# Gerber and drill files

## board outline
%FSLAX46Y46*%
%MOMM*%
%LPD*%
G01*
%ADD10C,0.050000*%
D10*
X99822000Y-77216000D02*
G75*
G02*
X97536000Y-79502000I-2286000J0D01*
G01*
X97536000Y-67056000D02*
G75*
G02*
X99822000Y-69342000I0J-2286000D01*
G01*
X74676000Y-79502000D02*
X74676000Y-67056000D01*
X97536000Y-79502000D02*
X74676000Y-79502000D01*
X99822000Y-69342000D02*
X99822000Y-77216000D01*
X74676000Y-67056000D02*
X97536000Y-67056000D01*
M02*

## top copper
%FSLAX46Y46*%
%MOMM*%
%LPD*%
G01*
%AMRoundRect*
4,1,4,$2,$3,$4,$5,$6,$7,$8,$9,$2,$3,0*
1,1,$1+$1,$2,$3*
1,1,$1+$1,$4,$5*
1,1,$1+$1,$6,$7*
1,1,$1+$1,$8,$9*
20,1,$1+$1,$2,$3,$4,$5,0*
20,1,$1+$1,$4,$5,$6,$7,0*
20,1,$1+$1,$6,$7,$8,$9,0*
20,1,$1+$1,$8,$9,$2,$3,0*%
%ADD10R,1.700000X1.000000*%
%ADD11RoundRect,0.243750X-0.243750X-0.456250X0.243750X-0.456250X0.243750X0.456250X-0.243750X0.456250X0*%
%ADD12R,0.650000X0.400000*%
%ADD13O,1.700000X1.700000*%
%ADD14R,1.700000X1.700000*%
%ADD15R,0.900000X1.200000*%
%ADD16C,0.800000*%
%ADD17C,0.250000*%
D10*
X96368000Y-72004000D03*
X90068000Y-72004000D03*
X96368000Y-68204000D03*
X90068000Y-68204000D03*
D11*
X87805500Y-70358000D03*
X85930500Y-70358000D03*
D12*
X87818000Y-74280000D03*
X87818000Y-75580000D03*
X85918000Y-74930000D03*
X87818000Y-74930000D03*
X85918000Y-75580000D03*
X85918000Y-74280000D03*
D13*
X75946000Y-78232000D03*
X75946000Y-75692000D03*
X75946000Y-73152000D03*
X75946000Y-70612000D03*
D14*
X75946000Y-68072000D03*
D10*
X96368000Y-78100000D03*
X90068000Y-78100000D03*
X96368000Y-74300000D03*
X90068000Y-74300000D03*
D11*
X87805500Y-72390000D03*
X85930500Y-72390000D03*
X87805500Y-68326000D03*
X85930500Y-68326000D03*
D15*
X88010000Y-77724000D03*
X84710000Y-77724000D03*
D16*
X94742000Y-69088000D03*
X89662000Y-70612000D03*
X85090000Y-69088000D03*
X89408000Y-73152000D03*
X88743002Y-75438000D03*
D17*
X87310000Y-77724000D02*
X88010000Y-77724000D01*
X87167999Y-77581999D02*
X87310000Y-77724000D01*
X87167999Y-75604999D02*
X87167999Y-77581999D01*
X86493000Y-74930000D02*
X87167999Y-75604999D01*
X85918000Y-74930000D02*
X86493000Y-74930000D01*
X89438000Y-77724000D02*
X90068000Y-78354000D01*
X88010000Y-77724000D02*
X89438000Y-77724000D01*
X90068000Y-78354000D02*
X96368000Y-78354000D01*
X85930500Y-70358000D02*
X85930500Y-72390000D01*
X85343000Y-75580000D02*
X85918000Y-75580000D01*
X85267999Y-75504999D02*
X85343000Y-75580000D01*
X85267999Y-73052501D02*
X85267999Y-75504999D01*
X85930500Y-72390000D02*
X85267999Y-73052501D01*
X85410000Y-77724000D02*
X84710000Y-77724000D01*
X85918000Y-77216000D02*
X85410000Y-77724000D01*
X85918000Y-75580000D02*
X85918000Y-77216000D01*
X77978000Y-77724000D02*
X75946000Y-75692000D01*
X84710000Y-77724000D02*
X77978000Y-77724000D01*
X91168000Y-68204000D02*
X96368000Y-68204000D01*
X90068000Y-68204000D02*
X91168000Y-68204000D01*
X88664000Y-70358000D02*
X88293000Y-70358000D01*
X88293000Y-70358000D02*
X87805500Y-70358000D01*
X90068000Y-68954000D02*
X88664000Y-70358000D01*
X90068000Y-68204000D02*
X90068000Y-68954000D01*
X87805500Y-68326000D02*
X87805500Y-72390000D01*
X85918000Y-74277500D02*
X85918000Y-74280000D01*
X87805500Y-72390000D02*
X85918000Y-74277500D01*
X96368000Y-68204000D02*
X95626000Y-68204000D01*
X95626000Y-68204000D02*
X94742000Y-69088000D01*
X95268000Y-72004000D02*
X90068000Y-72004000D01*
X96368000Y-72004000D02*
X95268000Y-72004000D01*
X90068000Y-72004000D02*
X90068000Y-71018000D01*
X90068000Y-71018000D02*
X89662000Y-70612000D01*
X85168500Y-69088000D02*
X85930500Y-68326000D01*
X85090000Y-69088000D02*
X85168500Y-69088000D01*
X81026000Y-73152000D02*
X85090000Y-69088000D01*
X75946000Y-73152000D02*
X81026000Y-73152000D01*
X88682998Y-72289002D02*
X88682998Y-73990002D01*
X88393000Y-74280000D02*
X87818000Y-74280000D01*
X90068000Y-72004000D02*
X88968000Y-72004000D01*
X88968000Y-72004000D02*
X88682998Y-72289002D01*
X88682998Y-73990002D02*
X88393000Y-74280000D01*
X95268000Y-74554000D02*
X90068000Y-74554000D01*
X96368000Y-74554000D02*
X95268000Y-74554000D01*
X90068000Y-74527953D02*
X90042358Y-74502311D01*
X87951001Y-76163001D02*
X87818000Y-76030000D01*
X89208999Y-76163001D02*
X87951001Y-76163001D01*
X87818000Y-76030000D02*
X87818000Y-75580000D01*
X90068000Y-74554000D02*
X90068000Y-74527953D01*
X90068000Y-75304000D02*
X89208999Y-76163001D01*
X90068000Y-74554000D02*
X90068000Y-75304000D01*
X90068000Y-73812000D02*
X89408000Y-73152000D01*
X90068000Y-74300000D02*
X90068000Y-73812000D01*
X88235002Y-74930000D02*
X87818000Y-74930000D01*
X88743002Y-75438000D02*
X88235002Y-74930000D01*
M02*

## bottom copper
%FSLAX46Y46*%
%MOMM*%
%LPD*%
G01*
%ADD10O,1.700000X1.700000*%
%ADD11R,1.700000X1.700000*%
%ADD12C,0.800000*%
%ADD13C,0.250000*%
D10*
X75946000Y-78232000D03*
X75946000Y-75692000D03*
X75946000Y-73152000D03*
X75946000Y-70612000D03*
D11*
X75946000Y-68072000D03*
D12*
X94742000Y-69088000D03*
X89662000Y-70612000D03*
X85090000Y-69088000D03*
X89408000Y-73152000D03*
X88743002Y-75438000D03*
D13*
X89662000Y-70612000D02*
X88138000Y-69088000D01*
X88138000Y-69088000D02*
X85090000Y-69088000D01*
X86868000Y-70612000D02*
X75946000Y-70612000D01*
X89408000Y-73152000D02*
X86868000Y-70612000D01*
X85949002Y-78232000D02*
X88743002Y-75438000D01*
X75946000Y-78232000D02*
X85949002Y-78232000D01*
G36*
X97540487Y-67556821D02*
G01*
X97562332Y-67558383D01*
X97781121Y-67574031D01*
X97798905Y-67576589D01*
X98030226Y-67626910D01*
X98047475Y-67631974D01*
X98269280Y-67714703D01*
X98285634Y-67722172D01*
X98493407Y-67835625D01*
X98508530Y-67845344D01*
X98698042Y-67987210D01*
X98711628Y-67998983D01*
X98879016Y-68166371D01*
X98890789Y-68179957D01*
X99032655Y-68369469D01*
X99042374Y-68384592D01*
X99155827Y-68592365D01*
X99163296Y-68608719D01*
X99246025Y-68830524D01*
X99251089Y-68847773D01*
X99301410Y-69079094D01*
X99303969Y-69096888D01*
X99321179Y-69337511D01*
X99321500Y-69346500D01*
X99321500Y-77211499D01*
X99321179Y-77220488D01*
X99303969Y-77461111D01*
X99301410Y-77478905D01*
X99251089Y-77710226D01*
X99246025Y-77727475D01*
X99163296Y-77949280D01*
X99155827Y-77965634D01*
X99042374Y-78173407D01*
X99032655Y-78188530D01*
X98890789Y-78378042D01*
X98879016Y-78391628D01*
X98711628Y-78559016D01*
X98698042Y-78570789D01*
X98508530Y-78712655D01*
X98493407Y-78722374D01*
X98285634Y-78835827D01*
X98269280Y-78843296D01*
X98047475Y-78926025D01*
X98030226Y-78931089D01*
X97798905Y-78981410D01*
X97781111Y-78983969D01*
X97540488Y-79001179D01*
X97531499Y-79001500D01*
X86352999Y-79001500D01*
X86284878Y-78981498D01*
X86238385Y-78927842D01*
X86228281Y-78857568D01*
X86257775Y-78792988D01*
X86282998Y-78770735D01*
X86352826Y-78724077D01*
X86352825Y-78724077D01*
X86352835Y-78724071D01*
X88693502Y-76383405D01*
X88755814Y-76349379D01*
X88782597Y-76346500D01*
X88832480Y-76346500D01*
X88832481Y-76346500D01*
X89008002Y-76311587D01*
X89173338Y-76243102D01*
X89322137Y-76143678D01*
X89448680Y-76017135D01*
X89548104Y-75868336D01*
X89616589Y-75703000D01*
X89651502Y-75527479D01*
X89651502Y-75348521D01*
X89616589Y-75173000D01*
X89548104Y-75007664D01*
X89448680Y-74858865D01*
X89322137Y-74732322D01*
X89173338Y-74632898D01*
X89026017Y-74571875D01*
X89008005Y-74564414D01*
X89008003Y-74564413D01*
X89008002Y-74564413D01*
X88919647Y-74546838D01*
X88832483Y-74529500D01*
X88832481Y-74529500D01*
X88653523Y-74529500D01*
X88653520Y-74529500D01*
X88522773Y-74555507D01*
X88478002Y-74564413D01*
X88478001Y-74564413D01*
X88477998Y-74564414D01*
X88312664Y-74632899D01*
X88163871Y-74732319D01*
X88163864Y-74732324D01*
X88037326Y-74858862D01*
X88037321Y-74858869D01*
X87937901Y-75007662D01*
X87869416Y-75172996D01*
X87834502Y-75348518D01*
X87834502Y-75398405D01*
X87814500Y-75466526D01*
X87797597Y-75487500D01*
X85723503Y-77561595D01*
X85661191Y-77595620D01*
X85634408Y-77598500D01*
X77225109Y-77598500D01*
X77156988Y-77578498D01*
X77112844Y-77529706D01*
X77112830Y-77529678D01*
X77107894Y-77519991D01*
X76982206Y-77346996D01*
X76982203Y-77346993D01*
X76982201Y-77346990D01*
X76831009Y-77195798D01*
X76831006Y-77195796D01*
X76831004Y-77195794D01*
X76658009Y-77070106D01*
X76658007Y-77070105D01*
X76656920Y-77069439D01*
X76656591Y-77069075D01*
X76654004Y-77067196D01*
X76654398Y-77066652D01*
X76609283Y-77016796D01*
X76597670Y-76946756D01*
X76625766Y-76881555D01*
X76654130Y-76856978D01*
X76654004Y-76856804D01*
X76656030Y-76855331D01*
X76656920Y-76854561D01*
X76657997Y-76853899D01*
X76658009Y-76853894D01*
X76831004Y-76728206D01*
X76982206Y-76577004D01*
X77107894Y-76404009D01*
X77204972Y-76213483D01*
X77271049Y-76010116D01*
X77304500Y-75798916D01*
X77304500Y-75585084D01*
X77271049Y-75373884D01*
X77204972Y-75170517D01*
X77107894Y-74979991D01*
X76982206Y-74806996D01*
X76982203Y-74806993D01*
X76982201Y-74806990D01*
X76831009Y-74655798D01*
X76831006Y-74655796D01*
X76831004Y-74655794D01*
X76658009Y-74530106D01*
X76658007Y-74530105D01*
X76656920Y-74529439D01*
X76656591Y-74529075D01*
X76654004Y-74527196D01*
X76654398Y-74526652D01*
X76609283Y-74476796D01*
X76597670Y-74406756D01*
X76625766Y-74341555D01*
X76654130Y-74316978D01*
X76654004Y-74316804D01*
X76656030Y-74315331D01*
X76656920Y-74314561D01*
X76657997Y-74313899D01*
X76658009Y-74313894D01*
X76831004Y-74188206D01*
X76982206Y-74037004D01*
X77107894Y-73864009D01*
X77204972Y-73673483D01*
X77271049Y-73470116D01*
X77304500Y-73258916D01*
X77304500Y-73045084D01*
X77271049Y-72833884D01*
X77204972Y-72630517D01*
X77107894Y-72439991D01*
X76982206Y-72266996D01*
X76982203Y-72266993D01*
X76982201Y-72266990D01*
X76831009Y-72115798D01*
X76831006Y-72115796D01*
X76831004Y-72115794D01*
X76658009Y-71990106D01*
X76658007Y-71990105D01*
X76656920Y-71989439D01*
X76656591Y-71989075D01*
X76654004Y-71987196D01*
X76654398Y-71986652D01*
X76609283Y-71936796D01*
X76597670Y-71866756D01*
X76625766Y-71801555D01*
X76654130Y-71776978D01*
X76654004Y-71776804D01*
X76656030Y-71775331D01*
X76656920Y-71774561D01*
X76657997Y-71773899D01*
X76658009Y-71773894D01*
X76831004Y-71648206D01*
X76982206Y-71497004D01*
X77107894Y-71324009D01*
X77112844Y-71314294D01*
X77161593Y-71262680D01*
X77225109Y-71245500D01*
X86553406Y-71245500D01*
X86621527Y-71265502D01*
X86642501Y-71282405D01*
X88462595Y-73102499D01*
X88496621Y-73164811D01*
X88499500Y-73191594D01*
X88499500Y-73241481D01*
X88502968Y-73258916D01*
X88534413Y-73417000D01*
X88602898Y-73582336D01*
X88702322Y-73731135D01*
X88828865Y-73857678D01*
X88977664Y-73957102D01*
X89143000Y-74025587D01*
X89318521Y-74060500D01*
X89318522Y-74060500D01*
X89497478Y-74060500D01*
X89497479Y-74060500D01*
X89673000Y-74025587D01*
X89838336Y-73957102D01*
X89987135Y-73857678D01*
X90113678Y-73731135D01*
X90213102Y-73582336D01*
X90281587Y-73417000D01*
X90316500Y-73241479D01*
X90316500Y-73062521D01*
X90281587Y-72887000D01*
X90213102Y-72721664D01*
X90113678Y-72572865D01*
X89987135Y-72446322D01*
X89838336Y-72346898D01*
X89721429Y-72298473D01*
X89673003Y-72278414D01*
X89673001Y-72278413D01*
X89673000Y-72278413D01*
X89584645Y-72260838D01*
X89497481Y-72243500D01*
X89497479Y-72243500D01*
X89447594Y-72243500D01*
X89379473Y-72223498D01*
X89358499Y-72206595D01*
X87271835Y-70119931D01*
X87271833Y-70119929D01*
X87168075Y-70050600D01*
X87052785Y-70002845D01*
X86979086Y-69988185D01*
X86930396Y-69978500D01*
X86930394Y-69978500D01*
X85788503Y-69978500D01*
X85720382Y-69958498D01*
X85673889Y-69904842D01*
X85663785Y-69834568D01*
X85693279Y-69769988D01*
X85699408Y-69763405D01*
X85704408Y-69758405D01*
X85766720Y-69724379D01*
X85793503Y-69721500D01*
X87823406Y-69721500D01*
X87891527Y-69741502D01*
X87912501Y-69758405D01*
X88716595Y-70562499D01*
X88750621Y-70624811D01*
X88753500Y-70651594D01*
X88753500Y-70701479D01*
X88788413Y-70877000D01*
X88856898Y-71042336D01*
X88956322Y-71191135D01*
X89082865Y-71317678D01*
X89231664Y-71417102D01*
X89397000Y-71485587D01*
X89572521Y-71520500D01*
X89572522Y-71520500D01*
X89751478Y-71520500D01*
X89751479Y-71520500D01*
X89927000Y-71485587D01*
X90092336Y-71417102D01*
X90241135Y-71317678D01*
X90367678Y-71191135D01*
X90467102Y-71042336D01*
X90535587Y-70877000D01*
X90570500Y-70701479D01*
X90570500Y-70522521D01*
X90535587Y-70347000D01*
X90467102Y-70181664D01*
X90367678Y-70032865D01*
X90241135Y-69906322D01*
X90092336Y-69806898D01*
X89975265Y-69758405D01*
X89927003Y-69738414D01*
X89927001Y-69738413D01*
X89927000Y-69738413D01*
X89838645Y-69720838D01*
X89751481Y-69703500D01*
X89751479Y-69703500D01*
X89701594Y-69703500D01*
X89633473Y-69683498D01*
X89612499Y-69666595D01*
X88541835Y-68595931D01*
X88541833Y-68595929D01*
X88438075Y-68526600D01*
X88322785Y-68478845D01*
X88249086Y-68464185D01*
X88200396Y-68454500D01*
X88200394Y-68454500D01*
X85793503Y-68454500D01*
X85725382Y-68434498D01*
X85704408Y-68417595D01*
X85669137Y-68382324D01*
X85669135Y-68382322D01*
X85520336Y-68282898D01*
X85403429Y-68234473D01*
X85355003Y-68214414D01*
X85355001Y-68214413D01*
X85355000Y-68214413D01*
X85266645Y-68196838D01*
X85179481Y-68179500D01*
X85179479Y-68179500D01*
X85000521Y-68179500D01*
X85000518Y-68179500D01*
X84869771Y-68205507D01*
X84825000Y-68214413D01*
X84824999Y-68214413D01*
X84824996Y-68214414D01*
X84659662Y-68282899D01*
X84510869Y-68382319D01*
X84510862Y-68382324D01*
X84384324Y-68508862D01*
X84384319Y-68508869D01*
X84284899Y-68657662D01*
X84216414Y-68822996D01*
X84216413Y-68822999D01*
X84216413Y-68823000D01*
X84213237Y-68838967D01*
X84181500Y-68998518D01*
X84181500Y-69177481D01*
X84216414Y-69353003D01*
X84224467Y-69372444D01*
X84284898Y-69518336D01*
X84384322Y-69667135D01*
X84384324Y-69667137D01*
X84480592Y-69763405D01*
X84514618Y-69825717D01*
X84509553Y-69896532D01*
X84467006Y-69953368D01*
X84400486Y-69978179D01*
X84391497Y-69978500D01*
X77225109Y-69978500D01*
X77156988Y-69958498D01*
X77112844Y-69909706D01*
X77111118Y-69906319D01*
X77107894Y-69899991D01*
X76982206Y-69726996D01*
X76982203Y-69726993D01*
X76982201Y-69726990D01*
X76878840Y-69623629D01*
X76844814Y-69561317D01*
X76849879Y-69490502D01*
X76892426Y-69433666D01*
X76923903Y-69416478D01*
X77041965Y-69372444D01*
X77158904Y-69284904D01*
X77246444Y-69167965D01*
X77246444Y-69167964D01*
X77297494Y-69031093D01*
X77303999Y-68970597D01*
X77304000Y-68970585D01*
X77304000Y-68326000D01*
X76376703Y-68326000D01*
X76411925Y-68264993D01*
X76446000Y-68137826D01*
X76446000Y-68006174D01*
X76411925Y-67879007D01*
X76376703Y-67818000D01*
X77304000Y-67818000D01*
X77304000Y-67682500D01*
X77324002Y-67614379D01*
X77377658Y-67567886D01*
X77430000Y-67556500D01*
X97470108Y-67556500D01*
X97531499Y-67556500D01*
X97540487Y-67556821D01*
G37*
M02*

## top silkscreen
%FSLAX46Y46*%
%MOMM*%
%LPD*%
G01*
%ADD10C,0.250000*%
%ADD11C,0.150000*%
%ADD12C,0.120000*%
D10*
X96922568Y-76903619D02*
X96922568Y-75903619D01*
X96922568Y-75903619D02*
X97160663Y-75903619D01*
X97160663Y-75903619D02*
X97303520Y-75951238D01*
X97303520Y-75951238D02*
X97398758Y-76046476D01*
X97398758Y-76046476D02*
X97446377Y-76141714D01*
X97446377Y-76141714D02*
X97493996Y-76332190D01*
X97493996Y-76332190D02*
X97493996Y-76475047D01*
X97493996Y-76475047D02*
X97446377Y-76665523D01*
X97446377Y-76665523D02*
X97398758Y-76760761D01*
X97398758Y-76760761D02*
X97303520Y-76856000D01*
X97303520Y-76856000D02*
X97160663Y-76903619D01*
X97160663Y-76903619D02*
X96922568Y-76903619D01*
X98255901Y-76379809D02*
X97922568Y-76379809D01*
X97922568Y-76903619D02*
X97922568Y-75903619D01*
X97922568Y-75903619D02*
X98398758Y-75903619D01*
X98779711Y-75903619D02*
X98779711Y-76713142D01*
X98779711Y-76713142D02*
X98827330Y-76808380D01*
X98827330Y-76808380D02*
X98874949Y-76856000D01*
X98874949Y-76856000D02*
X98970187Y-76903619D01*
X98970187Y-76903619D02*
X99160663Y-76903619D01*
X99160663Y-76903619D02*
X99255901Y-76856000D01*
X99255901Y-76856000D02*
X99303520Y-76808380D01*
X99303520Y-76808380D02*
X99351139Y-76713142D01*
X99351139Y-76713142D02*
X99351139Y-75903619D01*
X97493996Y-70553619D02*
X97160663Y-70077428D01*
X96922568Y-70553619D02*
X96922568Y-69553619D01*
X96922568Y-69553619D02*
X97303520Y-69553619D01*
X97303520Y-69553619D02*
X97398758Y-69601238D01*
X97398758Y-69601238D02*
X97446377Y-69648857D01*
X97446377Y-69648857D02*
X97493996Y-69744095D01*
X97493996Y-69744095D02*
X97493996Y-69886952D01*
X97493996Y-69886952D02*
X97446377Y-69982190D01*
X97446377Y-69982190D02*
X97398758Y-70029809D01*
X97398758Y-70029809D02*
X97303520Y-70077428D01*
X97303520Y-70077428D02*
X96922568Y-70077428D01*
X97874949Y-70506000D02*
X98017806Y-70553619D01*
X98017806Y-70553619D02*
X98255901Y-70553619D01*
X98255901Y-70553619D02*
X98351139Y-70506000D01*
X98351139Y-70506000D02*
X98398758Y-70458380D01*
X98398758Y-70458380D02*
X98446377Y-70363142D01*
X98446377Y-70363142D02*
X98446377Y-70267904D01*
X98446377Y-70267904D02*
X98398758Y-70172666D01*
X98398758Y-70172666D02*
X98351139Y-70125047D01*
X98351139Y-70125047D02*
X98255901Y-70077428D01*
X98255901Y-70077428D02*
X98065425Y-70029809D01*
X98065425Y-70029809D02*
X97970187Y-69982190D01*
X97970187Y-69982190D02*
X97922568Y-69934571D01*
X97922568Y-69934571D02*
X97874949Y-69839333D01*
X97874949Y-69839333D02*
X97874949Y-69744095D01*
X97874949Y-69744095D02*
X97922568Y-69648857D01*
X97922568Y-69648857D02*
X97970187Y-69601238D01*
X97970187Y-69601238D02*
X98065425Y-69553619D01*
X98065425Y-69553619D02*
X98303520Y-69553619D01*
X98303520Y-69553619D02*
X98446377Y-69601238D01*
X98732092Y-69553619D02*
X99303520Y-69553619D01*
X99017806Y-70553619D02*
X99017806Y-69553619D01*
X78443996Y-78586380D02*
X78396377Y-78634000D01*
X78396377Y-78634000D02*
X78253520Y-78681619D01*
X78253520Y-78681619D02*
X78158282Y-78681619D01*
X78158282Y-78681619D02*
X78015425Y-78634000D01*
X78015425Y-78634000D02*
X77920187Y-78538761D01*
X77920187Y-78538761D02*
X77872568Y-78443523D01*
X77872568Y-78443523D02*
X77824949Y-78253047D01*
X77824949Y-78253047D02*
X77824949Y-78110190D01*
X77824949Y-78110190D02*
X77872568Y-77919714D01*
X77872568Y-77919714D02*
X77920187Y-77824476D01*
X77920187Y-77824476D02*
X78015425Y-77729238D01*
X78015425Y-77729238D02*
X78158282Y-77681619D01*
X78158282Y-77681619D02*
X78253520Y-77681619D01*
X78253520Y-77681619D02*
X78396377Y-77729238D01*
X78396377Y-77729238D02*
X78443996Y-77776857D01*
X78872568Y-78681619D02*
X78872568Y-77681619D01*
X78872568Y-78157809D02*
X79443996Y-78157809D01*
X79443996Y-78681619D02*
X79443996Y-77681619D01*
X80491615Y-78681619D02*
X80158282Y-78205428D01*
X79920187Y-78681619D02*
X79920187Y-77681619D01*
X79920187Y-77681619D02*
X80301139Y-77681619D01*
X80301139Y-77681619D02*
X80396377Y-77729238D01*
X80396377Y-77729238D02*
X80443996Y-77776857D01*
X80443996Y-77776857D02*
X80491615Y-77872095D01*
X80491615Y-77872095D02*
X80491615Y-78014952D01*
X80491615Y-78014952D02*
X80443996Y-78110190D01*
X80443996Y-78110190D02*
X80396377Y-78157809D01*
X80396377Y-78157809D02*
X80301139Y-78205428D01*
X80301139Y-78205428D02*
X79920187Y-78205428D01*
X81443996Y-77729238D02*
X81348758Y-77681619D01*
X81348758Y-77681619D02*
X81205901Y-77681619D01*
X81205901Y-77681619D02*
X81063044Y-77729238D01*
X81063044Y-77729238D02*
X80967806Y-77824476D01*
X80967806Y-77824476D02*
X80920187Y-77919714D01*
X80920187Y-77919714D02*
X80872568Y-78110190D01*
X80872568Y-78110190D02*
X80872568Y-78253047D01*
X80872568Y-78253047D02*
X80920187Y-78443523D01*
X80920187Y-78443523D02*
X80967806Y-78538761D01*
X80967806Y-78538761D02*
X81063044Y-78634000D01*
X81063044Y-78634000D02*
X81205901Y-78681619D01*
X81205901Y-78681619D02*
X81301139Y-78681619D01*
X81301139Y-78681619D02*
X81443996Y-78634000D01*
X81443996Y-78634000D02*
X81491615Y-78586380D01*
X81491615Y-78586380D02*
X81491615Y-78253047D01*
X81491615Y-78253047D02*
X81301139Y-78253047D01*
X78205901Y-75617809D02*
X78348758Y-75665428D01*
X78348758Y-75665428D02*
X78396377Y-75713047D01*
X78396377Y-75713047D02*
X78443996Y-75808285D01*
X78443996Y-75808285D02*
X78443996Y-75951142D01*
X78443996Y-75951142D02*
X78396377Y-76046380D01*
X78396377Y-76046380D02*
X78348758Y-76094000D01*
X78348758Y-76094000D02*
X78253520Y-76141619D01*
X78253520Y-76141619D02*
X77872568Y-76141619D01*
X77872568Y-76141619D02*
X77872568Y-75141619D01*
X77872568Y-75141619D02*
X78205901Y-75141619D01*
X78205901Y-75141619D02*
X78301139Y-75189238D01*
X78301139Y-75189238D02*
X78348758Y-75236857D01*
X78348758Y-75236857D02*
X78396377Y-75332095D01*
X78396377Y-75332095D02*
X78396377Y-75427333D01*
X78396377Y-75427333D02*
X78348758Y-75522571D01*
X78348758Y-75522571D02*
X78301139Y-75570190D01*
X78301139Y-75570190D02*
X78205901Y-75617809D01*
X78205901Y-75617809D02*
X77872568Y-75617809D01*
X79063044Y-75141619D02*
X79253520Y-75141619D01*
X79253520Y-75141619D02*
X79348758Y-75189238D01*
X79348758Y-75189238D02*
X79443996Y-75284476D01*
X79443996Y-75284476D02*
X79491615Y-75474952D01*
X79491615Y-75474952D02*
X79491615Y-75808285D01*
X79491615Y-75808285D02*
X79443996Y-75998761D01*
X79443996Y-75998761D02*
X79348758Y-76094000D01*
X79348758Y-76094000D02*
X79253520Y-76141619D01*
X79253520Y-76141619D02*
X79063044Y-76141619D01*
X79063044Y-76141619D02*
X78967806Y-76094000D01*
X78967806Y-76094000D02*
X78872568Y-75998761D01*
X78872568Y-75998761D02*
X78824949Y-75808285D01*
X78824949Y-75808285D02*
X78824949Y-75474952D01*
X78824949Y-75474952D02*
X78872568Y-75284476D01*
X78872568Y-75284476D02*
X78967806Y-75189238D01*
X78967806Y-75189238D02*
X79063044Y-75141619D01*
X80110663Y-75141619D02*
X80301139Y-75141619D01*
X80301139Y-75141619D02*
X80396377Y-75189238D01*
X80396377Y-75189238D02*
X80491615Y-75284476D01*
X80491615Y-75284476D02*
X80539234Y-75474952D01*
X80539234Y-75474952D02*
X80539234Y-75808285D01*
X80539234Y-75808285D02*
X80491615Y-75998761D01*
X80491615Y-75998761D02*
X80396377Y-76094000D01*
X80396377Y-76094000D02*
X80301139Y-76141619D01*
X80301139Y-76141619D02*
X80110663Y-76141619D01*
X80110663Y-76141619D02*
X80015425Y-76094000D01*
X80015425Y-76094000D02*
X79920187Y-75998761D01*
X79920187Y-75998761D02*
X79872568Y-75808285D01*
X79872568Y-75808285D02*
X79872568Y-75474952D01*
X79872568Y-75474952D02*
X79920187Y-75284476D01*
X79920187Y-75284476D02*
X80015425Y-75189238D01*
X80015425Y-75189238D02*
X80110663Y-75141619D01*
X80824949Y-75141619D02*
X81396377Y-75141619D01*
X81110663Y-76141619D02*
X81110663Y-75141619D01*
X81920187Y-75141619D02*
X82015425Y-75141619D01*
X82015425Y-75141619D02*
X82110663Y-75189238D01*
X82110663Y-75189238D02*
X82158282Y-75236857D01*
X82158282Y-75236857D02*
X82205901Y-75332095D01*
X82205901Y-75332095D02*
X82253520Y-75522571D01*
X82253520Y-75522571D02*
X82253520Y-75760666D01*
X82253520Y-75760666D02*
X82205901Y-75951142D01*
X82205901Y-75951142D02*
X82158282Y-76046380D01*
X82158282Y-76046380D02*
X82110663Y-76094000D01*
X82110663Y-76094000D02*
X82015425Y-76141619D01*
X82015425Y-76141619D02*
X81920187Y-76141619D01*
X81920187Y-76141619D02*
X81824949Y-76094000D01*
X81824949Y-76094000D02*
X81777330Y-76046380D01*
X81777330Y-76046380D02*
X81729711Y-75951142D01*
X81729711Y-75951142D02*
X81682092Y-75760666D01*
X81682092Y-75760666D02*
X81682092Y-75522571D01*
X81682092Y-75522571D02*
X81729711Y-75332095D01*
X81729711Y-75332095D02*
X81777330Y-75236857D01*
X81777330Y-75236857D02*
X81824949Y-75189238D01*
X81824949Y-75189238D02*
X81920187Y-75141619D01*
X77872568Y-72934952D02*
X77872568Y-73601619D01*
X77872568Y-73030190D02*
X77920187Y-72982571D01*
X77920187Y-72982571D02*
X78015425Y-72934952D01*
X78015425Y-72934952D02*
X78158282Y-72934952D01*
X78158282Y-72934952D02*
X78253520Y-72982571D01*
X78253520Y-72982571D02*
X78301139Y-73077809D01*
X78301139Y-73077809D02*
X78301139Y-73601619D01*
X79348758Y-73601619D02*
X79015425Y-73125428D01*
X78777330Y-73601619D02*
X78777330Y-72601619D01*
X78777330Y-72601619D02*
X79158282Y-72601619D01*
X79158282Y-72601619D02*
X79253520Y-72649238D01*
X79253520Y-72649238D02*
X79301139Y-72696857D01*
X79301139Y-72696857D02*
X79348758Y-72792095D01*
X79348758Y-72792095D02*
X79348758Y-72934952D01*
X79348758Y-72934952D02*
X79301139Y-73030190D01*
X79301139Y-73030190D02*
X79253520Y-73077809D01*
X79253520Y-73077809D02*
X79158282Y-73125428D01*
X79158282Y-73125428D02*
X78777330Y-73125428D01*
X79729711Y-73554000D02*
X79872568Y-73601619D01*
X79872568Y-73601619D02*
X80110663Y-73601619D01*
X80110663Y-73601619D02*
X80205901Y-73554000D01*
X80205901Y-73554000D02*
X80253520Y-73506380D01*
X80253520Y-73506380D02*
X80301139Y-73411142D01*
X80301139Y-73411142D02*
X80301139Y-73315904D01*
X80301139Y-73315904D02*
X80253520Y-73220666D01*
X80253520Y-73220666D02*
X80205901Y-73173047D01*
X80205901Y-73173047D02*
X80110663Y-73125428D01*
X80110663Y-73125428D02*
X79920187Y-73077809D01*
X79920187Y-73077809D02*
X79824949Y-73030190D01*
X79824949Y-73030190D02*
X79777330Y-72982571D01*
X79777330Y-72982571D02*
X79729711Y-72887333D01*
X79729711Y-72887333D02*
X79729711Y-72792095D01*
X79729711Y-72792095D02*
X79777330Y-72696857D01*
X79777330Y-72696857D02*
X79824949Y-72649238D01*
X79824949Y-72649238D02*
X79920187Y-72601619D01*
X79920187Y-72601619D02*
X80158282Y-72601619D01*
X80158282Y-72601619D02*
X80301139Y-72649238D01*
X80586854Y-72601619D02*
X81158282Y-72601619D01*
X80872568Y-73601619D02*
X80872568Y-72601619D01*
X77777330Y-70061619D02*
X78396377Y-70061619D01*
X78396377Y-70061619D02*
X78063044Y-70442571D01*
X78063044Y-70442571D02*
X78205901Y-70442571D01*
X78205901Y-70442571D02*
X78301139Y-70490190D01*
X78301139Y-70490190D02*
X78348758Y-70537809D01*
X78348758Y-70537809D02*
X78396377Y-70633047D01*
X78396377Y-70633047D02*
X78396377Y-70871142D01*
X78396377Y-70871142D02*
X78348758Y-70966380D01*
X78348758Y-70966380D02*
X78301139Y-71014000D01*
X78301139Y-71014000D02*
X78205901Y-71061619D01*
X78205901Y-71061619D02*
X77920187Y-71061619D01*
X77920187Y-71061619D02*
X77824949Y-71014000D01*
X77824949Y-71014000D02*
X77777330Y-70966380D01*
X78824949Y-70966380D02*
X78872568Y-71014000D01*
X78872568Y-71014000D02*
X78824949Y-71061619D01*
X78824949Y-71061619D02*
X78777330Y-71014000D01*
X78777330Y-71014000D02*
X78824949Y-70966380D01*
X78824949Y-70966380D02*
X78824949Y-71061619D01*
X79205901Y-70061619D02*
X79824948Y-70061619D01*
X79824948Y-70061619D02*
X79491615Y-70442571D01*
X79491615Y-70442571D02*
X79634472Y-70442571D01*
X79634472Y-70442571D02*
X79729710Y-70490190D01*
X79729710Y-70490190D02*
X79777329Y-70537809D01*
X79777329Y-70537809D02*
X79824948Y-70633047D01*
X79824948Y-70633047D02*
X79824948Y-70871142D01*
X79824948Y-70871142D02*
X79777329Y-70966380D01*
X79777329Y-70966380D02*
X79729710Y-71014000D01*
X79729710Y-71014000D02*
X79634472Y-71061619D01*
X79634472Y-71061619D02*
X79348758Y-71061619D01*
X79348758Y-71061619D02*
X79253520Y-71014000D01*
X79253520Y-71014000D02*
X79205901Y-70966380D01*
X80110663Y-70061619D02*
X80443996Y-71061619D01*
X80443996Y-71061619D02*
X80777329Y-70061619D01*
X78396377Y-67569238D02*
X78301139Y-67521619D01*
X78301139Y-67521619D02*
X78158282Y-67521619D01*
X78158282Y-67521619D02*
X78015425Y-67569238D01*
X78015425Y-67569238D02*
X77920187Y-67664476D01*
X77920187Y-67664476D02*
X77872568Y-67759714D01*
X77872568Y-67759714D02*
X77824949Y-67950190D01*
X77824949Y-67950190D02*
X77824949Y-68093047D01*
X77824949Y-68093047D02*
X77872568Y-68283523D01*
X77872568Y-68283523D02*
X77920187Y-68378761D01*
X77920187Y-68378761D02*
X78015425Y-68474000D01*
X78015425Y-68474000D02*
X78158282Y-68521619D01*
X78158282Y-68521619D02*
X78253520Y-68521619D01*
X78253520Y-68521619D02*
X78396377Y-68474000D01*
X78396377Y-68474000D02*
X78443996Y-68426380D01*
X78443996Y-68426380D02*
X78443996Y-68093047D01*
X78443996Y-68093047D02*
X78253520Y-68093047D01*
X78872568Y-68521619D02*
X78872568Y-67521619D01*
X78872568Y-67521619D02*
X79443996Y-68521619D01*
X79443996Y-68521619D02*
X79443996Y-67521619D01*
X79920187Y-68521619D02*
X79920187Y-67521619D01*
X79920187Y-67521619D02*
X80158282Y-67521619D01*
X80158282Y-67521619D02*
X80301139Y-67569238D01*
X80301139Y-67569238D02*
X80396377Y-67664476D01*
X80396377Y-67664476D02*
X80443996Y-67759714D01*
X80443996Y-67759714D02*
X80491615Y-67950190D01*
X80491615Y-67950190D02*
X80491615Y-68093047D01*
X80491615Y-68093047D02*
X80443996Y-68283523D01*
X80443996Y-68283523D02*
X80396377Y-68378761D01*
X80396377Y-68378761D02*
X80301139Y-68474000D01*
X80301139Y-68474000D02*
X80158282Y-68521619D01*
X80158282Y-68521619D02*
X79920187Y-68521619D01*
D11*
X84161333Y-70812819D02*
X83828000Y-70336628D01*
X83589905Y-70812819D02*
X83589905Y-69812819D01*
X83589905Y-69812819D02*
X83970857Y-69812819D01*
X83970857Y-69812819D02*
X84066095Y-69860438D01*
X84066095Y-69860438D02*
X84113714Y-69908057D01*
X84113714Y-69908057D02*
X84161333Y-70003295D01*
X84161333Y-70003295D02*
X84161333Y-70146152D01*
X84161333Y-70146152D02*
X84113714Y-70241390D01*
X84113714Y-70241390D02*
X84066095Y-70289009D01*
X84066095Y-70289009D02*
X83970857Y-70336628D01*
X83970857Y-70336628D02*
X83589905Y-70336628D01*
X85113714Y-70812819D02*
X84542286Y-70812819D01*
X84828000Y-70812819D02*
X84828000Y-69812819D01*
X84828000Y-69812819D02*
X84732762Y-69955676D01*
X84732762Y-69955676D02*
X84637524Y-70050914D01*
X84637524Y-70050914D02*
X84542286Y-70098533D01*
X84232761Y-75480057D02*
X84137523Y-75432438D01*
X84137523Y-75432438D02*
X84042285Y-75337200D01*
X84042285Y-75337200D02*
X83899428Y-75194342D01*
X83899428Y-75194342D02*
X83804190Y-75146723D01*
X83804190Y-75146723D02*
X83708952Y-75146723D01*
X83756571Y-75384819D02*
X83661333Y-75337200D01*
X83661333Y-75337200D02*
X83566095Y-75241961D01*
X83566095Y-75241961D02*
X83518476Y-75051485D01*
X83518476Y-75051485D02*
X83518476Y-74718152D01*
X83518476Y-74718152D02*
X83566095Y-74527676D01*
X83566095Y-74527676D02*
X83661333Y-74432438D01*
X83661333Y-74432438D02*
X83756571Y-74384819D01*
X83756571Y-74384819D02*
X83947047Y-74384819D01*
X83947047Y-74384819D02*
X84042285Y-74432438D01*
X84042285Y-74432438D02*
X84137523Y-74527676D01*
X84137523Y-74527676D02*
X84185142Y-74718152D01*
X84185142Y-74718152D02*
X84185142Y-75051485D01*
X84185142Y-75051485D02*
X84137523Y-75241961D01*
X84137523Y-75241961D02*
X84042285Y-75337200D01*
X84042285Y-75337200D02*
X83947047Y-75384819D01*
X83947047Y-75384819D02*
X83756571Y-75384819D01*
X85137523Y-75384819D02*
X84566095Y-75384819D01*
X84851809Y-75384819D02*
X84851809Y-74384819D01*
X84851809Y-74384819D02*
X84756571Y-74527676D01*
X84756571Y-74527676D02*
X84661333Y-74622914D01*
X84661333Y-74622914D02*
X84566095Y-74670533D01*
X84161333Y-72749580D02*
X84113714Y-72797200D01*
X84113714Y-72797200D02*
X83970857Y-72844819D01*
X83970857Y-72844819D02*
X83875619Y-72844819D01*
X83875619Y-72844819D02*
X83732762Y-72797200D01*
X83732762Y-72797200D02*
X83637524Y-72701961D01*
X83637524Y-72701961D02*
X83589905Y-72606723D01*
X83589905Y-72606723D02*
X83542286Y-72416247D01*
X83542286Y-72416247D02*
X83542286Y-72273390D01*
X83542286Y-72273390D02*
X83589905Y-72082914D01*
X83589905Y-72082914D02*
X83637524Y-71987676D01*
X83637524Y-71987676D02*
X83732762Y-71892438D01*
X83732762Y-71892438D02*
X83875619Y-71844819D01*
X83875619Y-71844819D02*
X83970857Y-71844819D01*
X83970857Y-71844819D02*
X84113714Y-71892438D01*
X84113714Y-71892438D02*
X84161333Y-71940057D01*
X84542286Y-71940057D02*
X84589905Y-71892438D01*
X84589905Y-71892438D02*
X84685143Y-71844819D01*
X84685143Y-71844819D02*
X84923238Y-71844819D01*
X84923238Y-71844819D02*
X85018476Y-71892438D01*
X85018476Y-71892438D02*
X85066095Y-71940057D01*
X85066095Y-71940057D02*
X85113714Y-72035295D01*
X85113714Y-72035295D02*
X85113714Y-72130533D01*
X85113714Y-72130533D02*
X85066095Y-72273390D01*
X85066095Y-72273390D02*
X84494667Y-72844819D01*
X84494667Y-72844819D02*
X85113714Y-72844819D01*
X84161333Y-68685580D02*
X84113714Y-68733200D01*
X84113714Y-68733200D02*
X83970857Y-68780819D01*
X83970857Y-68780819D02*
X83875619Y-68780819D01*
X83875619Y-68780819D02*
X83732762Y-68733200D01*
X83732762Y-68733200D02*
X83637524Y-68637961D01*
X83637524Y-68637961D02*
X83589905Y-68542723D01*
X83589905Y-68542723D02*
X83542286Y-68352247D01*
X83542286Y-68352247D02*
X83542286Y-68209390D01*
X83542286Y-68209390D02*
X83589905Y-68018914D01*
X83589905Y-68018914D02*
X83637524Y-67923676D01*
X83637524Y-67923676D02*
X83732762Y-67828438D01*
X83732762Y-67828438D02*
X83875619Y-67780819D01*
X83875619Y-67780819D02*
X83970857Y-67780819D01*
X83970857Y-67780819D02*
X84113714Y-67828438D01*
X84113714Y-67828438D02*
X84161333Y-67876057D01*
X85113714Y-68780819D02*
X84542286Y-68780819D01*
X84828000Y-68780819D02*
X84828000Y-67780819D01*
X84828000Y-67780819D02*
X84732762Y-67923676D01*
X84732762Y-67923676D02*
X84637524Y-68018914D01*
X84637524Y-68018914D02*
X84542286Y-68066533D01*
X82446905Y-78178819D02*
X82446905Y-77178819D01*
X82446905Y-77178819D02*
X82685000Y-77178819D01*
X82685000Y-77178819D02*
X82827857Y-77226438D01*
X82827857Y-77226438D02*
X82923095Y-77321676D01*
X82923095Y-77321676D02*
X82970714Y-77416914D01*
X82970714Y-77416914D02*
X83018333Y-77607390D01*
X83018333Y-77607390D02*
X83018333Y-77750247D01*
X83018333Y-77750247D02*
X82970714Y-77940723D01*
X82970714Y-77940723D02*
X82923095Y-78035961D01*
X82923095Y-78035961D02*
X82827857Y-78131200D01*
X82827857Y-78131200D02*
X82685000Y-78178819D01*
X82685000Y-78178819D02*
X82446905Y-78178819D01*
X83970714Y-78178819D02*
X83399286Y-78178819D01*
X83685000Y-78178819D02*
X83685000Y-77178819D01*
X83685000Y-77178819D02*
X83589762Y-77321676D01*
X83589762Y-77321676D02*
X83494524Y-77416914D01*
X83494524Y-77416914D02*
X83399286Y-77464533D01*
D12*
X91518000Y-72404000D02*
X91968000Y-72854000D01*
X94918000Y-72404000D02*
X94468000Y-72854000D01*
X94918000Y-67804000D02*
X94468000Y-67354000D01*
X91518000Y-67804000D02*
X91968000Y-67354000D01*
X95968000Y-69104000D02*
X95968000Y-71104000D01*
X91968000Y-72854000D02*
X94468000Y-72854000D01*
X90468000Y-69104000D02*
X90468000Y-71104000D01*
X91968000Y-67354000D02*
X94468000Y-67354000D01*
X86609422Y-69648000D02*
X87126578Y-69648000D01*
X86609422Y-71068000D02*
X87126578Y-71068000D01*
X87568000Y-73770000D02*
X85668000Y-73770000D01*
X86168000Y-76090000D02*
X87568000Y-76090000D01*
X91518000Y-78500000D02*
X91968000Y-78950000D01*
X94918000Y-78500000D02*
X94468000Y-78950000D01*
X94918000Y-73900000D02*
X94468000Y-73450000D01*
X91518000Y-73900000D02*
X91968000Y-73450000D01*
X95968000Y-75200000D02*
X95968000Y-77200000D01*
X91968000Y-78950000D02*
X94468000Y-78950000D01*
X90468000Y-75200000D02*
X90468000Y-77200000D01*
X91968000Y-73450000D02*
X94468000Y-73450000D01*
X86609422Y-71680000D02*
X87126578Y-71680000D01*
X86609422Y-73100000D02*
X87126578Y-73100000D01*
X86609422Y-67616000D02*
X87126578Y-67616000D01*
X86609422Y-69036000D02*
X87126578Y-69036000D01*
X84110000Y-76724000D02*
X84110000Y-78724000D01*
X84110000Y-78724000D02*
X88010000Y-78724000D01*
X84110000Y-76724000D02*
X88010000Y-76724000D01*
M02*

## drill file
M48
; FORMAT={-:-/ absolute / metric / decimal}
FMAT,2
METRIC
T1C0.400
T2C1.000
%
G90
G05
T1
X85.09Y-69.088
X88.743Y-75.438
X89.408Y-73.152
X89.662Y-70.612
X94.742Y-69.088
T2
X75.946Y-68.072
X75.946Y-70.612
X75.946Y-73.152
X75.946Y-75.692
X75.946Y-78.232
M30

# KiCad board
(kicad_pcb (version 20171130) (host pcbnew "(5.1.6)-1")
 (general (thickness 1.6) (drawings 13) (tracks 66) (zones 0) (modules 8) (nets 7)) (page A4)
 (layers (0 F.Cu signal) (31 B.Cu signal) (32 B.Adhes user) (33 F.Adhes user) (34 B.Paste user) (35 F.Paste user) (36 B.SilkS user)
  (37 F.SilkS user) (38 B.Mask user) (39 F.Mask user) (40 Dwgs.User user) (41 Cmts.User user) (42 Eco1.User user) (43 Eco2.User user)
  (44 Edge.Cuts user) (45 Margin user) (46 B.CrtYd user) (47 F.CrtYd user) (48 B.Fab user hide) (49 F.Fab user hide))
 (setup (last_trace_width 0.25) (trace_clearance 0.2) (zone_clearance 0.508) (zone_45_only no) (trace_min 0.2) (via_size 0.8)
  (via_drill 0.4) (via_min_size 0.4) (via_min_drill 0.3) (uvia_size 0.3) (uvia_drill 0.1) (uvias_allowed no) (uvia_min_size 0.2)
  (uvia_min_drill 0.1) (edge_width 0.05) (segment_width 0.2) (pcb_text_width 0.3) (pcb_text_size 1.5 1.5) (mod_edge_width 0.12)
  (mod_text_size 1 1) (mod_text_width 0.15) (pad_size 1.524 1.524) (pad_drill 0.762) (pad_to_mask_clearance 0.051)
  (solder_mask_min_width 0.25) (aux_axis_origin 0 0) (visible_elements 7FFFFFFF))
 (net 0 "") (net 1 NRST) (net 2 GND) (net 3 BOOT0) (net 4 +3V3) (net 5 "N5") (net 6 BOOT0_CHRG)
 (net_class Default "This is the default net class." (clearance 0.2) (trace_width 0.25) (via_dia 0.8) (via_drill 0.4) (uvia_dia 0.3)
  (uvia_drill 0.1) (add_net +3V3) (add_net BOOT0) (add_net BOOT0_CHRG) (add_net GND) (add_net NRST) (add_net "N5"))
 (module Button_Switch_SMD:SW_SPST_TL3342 (layer F.Cu) (at 93.218 70.104)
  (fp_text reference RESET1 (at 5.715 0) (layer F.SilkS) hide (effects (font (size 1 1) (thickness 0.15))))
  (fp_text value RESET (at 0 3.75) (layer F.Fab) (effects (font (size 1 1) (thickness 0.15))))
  (fp_line (start -1.7 2.3) (end -1.25 2.75) (layer F.SilkS) (width 0.12))
  (fp_line (start 1.7 2.3) (end 1.25 2.75) (layer F.SilkS) (width 0.12))
  (fp_line (start 1.7 -2.3) (end 1.25 -2.75) (layer F.SilkS) (width 0.12))
  (fp_line (start -1.7 -2.3) (end -1.25 -2.75) (layer F.SilkS) (width 0.12))
  (fp_line (start 2.75 -1) (end 2.75 1) (layer F.SilkS) (width 0.12))
  (fp_line (start -1.25 2.75) (end 1.25 2.75) (layer F.SilkS) (width 0.12))
  (fp_line (start -2.75 -1) (end -2.75 1) (layer F.SilkS) (width 0.12))
  (fp_line (start -1.25 -2.75) (end 1.25 -2.75) (layer F.SilkS) (width 0.12))
  (pad 2 smd rect (at 3.15 1.9) (size 1.7 1) (layers F.Cu F.Paste F.Mask) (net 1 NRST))
  (pad 2 smd rect (at -3.15 1.9) (size 1.7 1) (layers F.Cu F.Paste F.Mask) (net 1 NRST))
  (pad 1 smd rect (at 3.15 -1.9) (size 1.7 1) (layers F.Cu F.Paste F.Mask) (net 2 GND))
  (pad 1 smd rect (at -3.15 -1.9) (size 1.7 1) (layers F.Cu F.Paste F.Mask) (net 2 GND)))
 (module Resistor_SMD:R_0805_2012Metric (layer F.Cu) (at 86.868 70.358)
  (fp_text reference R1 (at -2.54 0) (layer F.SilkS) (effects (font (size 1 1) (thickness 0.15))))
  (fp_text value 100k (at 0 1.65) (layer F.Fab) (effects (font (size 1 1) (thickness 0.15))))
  (fp_line (start -0.258578 -0.71) (end 0.258578 -0.71) (layer F.SilkS) (width 0.12))
  (fp_line (start -0.258578 0.71) (end 0.258578 0.71) (layer F.SilkS) (width 0.12))
  (pad 2 smd roundrect (at 0.9375 0) (size 0.975 1.4) (layers F.Cu F.Paste F.Mask) (roundrect_rratio 0.25) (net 2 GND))
  (pad 1 smd roundrect (at -0.9375 0) (size 0.975 1.4) (layers F.Cu F.Paste F.Mask) (roundrect_rratio 0.25) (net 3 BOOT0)))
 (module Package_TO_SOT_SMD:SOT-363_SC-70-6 (layer F.Cu) (at 86.868 74.93)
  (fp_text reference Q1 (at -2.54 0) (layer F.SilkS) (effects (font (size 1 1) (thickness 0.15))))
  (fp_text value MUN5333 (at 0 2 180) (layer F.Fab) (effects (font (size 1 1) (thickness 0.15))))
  (fp_line (start 0.7 -1.16) (end -1.2 -1.16) (layer F.SilkS) (width 0.12))
  (fp_line (start -0.7 1.16) (end 0.7 1.16) (layer F.SilkS) (width 0.12))
  (pad 6 smd rect (at 0.95 -0.65) (size 0.65 0.4) (layers F.Cu F.Paste F.Mask) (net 1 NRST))
  (pad 4 smd rect (at 0.95 0.65) (size 0.65 0.4) (layers F.Cu F.Paste F.Mask) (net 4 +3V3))
  (pad 2 smd rect (at -0.95 0) (size 0.65 0.4) (layers F.Cu F.Paste F.Mask) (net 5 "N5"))
  (pad 5 smd rect (at 0.95 0) (size 0.65 0.4) (layers F.Cu F.Paste F.Mask) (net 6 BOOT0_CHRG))
  (pad 3 smd rect (at -0.95 0.65) (size 0.65 0.4) (layers F.Cu F.Paste F.Mask) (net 3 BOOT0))
  (pad 1 smd rect (at -0.95 -0.65) (size 0.65 0.4) (layers F.Cu F.Paste F.Mask) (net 2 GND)))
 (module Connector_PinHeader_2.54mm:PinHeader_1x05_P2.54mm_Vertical (layer B.Cu) (at 75.946 68.072 180)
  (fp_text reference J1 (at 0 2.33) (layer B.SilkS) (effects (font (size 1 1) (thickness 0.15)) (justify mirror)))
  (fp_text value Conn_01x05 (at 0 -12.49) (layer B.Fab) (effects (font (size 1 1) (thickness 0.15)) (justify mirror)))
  (pad 5 thru_hole oval (at 0 -10.16 180) (size 1.7 1.7) (drill 1) (layers *.Cu *.Mask) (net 6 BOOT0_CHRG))
  (pad 4 thru_hole oval (at 0 -7.62 180) (size 1.7 1.7) (drill 1) (layers *.Cu *.Mask) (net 3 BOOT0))
  (pad 3 thru_hole oval (at 0 -5.08 180) (size 1.7 1.7) (drill 1) (layers *.Cu *.Mask) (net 1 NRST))
  (pad 2 thru_hole oval (at 0 -2.54 180) (size 1.7 1.7) (drill 1) (layers *.Cu *.Mask) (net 4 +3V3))
  (pad 1 thru_hole rect (at 0 0 180) (size 1.7 1.7) (drill 1) (layers *.Cu *.Mask) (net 2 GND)))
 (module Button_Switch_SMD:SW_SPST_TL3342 (layer F.Cu) (at 93.218 76.2)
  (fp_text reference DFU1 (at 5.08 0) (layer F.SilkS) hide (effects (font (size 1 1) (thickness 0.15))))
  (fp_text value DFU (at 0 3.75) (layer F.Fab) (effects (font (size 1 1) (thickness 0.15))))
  (fp_line (start -1.7 2.3) (end -1.25 2.75) (layer F.SilkS) (width 0.12))
  (fp_line (start 1.7 2.3) (end 1.25 2.75) (layer F.SilkS) (width 0.12))
  (fp_line (start 1.7 -2.3) (end 1.25 -2.75) (layer F.SilkS) (width 0.12))
  (fp_line (start -1.7 -2.3) (end -1.25 -2.75) (layer F.SilkS) (width 0.12))
  (fp_line (start 2.75 -1) (end 2.75 1) (layer F.SilkS) (width 0.12))
  (fp_line (start -1.25 2.75) (end 1.25 2.75) (layer F.SilkS) (width 0.12))
  (fp_line (start -2.75 -1) (end -2.75 1) (layer F.SilkS) (width 0.12))
  (fp_line (start -1.25 -2.75) (end 1.25 -2.75) (layer F.SilkS) (width 0.12))
  (pad 2 smd rect (at 3.15 1.9) (size 1.7 1) (layers F.Cu F.Paste F.Mask) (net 5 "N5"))
  (pad 2 smd rect (at -3.15 1.9) (size 1.7 1) (layers F.Cu F.Paste F.Mask) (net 5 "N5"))
  (pad 1 smd rect (at 3.15 -1.9) (size 1.7 1) (layers F.Cu F.Paste F.Mask) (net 4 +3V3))
  (pad 1 smd rect (at -3.15 -1.9) (size 1.7 1) (layers F.Cu F.Paste F.Mask) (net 4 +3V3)))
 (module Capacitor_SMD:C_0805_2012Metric (layer F.Cu) (at 86.868 72.39)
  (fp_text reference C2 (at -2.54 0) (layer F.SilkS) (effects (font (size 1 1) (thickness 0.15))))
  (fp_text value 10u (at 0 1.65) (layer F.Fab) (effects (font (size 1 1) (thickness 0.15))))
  (fp_line (start -0.258578 -0.71) (end 0.258578 -0.71) (layer F.SilkS) (width 0.12))
  (fp_line (start -0.258578 0.71) (end 0.258578 0.71) (layer F.SilkS) (width 0.12))
  (pad 2 smd roundrect (at 0.9375 0) (size 0.975 1.4) (layers F.Cu F.Paste F.Mask) (roundrect_rratio 0.25) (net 2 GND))
  (pad 1 smd roundrect (at -0.9375 0) (size 0.975 1.4) (layers F.Cu F.Paste F.Mask) (roundrect_rratio 0.25) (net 3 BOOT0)))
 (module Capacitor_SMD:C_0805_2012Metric (layer F.Cu) (at 86.868 68.326)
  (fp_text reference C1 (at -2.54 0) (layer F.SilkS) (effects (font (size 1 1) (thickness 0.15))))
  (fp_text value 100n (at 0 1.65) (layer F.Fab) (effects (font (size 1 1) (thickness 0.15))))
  (fp_line (start -0.258578 -0.71) (end 0.258578 -0.71) (layer F.SilkS) (width 0.12))
  (fp_line (start -0.258578 0.71) (end 0.258578 0.71) (layer F.SilkS) (width 0.12))
  (pad 2 smd roundrect (at 0.9375 0) (size 0.975 1.4) (layers F.Cu F.Paste F.Mask) (roundrect_rratio 0.25) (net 2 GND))
  (pad 1 smd roundrect (at -0.9375 0) (size 0.975 1.4) (layers F.Cu F.Paste F.Mask) (roundrect_rratio 0.25) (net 1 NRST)))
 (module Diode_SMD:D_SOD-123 (layer F.Cu) (at 86.36 77.724)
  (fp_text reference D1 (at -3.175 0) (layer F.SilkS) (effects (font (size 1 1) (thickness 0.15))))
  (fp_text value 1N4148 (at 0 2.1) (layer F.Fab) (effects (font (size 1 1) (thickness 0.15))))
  (fp_line (start -2.25 -1) (end -2.25 1) (layer F.SilkS) (width 0.12))
  (fp_line (start -2.25 1) (end 1.65 1) (layer F.SilkS) (width 0.12))
  (fp_line (start -2.25 -1) (end 1.65 -1) (layer F.SilkS) (width 0.12))
  (pad 2 smd rect (at 1.65 0) (size 0.9 1.2) (layers F.Cu F.Paste F.Mask) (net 5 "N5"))
  (pad 1 smd rect (at -1.65 0) (size 0.9 1.2) (layers F.Cu F.Paste F.Mask) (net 3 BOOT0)))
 (gr_arc (start 97.536 77.216) (end 97.536 79.502) (angle -90) (layer Edge.Cuts) (width 0.05))
 (gr_arc (start 97.536 69.342) (end 99.822 69.342) (angle -90) (layer Edge.Cuts) (width 0.05))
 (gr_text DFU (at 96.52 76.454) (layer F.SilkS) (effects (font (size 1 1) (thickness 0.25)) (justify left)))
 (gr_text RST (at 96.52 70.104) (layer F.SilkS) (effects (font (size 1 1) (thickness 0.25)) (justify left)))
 (gr_line (start 74.676 79.502) (end 74.676 67.056) (layer Edge.Cuts) (width 0.05))
 (gr_line (start 97.536 79.502) (end 74.676 79.502) (layer Edge.Cuts) (width 0.05))
 (gr_line (start 99.822 69.342) (end 99.822 77.216) (layer Edge.Cuts) (width 0.05))
 (gr_line (start 74.676 67.056) (end 97.536 67.056) (layer Edge.Cuts) (width 0.05))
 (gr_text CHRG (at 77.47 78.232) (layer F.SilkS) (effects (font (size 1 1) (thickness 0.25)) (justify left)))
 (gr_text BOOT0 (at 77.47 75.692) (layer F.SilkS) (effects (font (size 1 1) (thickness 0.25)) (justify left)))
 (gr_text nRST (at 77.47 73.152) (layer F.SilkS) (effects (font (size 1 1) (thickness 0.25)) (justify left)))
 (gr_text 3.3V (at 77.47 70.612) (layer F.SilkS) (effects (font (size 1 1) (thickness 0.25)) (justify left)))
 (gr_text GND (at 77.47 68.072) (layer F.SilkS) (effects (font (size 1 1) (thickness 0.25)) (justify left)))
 (segment (start 87.31 77.724) (end 88.01 77.724) (width 0.25) (layer F.Cu) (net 5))
 (segment (start 87.167999 77.581999) (end 87.31 77.724) (width 0.25) (layer F.Cu) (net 5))
 (segment (start 87.167999 75.604999) (end 87.167999 77.581999) (width 0.25) (layer F.Cu) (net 5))
 (segment (start 86.493 74.93) (end 87.167999 75.604999) (width 0.25) (layer F.Cu) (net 5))
 (segment (start 85.918 74.93) (end 86.493 74.93) (width 0.25) (layer F.Cu) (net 5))
 (segment (start 89.438 77.724) (end 90.068 78.354) (width 0.25) (layer F.Cu) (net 5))
 (segment (start 88.01 77.724) (end 89.438 77.724) (width 0.25) (layer F.Cu) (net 5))
 (segment (start 90.068 78.354) (end 96.368 78.354) (width 0.25) (layer F.Cu) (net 5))
 (segment (start 85.9305 70.358) (end 85.9305 72.39) (width 0.25) (layer F.Cu) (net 3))
 (segment (start 85.343 75.58) (end 85.918 75.58) (width 0.25) (layer F.Cu) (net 3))
 (segment (start 85.267999 75.504999) (end 85.343 75.58) (width 0.25) (layer F.Cu) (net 3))
 (segment (start 85.267999 73.052501) (end 85.267999 75.504999) (width 0.25) (layer F.Cu) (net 3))
 (segment (start 85.9305 72.39) (end 85.267999 73.052501) (width 0.25) (layer F.Cu) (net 3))
 (segment (start 85.41 77.724) (end 84.71 77.724) (width 0.25) (layer F.Cu) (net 3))
 (segment (start 85.918 77.216) (end 85.41 77.724) (width 0.25) (layer F.Cu) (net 3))
 (segment (start 85.918 75.58) (end 85.918 77.216) (width 0.25) (layer F.Cu) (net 3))
 (segment (start 77.978 77.724) (end 75.946 75.692) (width 0.25) (layer F.Cu) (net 3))
 (segment (start 84.71 77.724) (end 77.978 77.724) (width 0.25) (layer F.Cu) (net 3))
 (segment (start 91.168 68.204) (end 96.368 68.204) (width 0.25) (layer F.Cu) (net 2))
 (segment (start 90.068 68.204) (end 91.168 68.204) (width 0.25) (layer F.Cu) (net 2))
 (segment (start 88.664 70.358) (end 88.293 70.358) (width 0.25) (layer F.Cu) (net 2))
 (segment (start 88.293 70.358) (end 87.8055 70.358) (width 0.25) (layer F.Cu) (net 2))
 (segment (start 90.068 68.954) (end 88.664 70.358) (width 0.25) (layer F.Cu) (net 2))
 (segment (start 90.068 68.204) (end 90.068 68.954) (width 0.25) (layer F.Cu) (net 2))
 (segment (start 87.8055 68.326) (end 87.8055 72.39) (width 0.25) (layer F.Cu) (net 2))
 (segment (start 85.918 74.2775) (end 85.918 74.28) (width 0.25) (layer F.Cu) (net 2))
 (segment (start 87.8055 72.39) (end 85.918 74.2775) (width 0.25) (layer F.Cu) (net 2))
 (via (at 94.742 69.088) (size 0.8) (drill 0.4) (layers F.Cu B.Cu) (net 2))
 (segment (start 96.368 68.204) (end 95.626 68.204) (width 0.25) (layer F.Cu) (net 2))
 (segment (start 95.626 68.204) (end 94.742 69.088) (width 0.25) (layer F.Cu) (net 2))
 (segment (start 95.268 72.004) (end 90.068 72.004) (width 0.25) (layer F.Cu) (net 1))
 (segment (start 96.368 72.004) (end 95.268 72.004) (width 0.25) (layer F.Cu) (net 1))
 (via (at 89.662 70.612) (size 0.8) (drill 0.4) (layers F.Cu B.Cu) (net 1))
 (segment (start 90.068 72.004) (end 90.068 71.018) (width 0.25) (layer F.Cu) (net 1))
 (segment (start 90.068 71.018) (end 89.662 70.612) (width 0.25) (layer F.Cu) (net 1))
 (via (at 85.09 69.088) (size 0.8) (drill 0.4) (layers F.Cu B.Cu) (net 1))
 (segment (start 89.662 70.612) (end 88.138 69.088) (width 0.25) (layer B.Cu) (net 1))
 (segment (start 88.138 69.088) (end 85.09 69.088) (width 0.25) (layer B.Cu) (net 1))
 (segment (start 85.1685 69.088) (end 85.9305 68.326) (width 0.25) (layer F.Cu) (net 1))
 (segment (start 85.09 69.088) (end 85.1685 69.088) (width 0.25) (layer F.Cu) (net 1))
 (segment (start 81.026 73.152) (end 85.09 69.088) (width 0.25) (layer F.Cu) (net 1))
 (segment (start 75.946 73.152) (end 81.026 73.152) (width 0.25) (layer F.Cu) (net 1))
 (segment (start 88.682998 72.289002) (end 88.682998 73.990002) (width 0.25) (layer F.Cu) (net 1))
 (segment (start 88.393 74.28) (end 87.818 74.28) (width 0.25) (layer F.Cu) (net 1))
 (segment (start 90.068 72.004) (end 88.968 72.004) (width 0.25) (layer F.Cu) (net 1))
 (segment (start 88.968 72.004) (end 88.682998 72.289002) (width 0.25) (layer F.Cu) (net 1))
 (segment (start 88.682998 73.990002) (end 88.393 74.28) (width 0.25) (layer F.Cu) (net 1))
 (segment (start 95.268 74.554) (end 90.068 74.554) (width 0.25) (layer F.Cu) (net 4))
 (segment (start 96.368 74.554) (end 95.268 74.554) (width 0.25) (layer F.Cu) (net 4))
 (segment (start 90.068 74.527953) (end 90.042358 74.502311) (width 0.25) (layer F.Cu) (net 4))
 (segment (start 87.951001 76.163001) (end 87.818 76.03) (width 0.25) (layer F.Cu) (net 4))
 (segment (start 89.208999 76.163001) (end 87.951001 76.163001) (width 0.25) (layer F.Cu) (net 4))
 (segment (start 87.818 76.03) (end 87.818 75.58) (width 0.25) (layer F.Cu) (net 4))
 (segment (start 90.068 74.554) (end 90.068 74.527953) (width 0.25) (layer F.Cu) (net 4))
 (segment (start 90.068 75.304) (end 89.208999 76.163001) (width 0.25) (layer F.Cu) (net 4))
 (segment (start 90.068 74.554) (end 90.068 75.304) (width 0.25) (layer F.Cu) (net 4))
 (via (at 89.408 73.152) (size 0.8) (drill 0.4) (layers F.Cu B.Cu) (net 4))
 (segment (start 90.068 73.812) (end 89.408 73.152) (width 0.25) (layer F.Cu) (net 4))
 (segment (start 90.068 74.3) (end 90.068 73.812) (width 0.25) (layer F.Cu) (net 4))
 (segment (start 86.868 70.612) (end 75.946 70.612) (width 0.25) (layer B.Cu) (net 4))
 (segment (start 89.408 73.152) (end 86.868 70.612) (width 0.25) (layer B.Cu) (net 4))
 (via (at 88.743002 75.438) (size 0.8) (drill 0.4) (layers F.Cu B.Cu) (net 6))
 (segment (start 85.949002 78.232) (end 88.743002 75.438) (width 0.25) (layer B.Cu) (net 6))
 (segment (start 75.946 78.232) (end 85.949002 78.232) (width 0.25) (layer B.Cu) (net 6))
 (segment (start 88.235002 74.93) (end 87.818 74.93) (width 0.25) (layer F.Cu) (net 6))
 (segment (start 88.743002 75.438) (end 88.235002 74.93) (width 0.25) (layer F.Cu) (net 6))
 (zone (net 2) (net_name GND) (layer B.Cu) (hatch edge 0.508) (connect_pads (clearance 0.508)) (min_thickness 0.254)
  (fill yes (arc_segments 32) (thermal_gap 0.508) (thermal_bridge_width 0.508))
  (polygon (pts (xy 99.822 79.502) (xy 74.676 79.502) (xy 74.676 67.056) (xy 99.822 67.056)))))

